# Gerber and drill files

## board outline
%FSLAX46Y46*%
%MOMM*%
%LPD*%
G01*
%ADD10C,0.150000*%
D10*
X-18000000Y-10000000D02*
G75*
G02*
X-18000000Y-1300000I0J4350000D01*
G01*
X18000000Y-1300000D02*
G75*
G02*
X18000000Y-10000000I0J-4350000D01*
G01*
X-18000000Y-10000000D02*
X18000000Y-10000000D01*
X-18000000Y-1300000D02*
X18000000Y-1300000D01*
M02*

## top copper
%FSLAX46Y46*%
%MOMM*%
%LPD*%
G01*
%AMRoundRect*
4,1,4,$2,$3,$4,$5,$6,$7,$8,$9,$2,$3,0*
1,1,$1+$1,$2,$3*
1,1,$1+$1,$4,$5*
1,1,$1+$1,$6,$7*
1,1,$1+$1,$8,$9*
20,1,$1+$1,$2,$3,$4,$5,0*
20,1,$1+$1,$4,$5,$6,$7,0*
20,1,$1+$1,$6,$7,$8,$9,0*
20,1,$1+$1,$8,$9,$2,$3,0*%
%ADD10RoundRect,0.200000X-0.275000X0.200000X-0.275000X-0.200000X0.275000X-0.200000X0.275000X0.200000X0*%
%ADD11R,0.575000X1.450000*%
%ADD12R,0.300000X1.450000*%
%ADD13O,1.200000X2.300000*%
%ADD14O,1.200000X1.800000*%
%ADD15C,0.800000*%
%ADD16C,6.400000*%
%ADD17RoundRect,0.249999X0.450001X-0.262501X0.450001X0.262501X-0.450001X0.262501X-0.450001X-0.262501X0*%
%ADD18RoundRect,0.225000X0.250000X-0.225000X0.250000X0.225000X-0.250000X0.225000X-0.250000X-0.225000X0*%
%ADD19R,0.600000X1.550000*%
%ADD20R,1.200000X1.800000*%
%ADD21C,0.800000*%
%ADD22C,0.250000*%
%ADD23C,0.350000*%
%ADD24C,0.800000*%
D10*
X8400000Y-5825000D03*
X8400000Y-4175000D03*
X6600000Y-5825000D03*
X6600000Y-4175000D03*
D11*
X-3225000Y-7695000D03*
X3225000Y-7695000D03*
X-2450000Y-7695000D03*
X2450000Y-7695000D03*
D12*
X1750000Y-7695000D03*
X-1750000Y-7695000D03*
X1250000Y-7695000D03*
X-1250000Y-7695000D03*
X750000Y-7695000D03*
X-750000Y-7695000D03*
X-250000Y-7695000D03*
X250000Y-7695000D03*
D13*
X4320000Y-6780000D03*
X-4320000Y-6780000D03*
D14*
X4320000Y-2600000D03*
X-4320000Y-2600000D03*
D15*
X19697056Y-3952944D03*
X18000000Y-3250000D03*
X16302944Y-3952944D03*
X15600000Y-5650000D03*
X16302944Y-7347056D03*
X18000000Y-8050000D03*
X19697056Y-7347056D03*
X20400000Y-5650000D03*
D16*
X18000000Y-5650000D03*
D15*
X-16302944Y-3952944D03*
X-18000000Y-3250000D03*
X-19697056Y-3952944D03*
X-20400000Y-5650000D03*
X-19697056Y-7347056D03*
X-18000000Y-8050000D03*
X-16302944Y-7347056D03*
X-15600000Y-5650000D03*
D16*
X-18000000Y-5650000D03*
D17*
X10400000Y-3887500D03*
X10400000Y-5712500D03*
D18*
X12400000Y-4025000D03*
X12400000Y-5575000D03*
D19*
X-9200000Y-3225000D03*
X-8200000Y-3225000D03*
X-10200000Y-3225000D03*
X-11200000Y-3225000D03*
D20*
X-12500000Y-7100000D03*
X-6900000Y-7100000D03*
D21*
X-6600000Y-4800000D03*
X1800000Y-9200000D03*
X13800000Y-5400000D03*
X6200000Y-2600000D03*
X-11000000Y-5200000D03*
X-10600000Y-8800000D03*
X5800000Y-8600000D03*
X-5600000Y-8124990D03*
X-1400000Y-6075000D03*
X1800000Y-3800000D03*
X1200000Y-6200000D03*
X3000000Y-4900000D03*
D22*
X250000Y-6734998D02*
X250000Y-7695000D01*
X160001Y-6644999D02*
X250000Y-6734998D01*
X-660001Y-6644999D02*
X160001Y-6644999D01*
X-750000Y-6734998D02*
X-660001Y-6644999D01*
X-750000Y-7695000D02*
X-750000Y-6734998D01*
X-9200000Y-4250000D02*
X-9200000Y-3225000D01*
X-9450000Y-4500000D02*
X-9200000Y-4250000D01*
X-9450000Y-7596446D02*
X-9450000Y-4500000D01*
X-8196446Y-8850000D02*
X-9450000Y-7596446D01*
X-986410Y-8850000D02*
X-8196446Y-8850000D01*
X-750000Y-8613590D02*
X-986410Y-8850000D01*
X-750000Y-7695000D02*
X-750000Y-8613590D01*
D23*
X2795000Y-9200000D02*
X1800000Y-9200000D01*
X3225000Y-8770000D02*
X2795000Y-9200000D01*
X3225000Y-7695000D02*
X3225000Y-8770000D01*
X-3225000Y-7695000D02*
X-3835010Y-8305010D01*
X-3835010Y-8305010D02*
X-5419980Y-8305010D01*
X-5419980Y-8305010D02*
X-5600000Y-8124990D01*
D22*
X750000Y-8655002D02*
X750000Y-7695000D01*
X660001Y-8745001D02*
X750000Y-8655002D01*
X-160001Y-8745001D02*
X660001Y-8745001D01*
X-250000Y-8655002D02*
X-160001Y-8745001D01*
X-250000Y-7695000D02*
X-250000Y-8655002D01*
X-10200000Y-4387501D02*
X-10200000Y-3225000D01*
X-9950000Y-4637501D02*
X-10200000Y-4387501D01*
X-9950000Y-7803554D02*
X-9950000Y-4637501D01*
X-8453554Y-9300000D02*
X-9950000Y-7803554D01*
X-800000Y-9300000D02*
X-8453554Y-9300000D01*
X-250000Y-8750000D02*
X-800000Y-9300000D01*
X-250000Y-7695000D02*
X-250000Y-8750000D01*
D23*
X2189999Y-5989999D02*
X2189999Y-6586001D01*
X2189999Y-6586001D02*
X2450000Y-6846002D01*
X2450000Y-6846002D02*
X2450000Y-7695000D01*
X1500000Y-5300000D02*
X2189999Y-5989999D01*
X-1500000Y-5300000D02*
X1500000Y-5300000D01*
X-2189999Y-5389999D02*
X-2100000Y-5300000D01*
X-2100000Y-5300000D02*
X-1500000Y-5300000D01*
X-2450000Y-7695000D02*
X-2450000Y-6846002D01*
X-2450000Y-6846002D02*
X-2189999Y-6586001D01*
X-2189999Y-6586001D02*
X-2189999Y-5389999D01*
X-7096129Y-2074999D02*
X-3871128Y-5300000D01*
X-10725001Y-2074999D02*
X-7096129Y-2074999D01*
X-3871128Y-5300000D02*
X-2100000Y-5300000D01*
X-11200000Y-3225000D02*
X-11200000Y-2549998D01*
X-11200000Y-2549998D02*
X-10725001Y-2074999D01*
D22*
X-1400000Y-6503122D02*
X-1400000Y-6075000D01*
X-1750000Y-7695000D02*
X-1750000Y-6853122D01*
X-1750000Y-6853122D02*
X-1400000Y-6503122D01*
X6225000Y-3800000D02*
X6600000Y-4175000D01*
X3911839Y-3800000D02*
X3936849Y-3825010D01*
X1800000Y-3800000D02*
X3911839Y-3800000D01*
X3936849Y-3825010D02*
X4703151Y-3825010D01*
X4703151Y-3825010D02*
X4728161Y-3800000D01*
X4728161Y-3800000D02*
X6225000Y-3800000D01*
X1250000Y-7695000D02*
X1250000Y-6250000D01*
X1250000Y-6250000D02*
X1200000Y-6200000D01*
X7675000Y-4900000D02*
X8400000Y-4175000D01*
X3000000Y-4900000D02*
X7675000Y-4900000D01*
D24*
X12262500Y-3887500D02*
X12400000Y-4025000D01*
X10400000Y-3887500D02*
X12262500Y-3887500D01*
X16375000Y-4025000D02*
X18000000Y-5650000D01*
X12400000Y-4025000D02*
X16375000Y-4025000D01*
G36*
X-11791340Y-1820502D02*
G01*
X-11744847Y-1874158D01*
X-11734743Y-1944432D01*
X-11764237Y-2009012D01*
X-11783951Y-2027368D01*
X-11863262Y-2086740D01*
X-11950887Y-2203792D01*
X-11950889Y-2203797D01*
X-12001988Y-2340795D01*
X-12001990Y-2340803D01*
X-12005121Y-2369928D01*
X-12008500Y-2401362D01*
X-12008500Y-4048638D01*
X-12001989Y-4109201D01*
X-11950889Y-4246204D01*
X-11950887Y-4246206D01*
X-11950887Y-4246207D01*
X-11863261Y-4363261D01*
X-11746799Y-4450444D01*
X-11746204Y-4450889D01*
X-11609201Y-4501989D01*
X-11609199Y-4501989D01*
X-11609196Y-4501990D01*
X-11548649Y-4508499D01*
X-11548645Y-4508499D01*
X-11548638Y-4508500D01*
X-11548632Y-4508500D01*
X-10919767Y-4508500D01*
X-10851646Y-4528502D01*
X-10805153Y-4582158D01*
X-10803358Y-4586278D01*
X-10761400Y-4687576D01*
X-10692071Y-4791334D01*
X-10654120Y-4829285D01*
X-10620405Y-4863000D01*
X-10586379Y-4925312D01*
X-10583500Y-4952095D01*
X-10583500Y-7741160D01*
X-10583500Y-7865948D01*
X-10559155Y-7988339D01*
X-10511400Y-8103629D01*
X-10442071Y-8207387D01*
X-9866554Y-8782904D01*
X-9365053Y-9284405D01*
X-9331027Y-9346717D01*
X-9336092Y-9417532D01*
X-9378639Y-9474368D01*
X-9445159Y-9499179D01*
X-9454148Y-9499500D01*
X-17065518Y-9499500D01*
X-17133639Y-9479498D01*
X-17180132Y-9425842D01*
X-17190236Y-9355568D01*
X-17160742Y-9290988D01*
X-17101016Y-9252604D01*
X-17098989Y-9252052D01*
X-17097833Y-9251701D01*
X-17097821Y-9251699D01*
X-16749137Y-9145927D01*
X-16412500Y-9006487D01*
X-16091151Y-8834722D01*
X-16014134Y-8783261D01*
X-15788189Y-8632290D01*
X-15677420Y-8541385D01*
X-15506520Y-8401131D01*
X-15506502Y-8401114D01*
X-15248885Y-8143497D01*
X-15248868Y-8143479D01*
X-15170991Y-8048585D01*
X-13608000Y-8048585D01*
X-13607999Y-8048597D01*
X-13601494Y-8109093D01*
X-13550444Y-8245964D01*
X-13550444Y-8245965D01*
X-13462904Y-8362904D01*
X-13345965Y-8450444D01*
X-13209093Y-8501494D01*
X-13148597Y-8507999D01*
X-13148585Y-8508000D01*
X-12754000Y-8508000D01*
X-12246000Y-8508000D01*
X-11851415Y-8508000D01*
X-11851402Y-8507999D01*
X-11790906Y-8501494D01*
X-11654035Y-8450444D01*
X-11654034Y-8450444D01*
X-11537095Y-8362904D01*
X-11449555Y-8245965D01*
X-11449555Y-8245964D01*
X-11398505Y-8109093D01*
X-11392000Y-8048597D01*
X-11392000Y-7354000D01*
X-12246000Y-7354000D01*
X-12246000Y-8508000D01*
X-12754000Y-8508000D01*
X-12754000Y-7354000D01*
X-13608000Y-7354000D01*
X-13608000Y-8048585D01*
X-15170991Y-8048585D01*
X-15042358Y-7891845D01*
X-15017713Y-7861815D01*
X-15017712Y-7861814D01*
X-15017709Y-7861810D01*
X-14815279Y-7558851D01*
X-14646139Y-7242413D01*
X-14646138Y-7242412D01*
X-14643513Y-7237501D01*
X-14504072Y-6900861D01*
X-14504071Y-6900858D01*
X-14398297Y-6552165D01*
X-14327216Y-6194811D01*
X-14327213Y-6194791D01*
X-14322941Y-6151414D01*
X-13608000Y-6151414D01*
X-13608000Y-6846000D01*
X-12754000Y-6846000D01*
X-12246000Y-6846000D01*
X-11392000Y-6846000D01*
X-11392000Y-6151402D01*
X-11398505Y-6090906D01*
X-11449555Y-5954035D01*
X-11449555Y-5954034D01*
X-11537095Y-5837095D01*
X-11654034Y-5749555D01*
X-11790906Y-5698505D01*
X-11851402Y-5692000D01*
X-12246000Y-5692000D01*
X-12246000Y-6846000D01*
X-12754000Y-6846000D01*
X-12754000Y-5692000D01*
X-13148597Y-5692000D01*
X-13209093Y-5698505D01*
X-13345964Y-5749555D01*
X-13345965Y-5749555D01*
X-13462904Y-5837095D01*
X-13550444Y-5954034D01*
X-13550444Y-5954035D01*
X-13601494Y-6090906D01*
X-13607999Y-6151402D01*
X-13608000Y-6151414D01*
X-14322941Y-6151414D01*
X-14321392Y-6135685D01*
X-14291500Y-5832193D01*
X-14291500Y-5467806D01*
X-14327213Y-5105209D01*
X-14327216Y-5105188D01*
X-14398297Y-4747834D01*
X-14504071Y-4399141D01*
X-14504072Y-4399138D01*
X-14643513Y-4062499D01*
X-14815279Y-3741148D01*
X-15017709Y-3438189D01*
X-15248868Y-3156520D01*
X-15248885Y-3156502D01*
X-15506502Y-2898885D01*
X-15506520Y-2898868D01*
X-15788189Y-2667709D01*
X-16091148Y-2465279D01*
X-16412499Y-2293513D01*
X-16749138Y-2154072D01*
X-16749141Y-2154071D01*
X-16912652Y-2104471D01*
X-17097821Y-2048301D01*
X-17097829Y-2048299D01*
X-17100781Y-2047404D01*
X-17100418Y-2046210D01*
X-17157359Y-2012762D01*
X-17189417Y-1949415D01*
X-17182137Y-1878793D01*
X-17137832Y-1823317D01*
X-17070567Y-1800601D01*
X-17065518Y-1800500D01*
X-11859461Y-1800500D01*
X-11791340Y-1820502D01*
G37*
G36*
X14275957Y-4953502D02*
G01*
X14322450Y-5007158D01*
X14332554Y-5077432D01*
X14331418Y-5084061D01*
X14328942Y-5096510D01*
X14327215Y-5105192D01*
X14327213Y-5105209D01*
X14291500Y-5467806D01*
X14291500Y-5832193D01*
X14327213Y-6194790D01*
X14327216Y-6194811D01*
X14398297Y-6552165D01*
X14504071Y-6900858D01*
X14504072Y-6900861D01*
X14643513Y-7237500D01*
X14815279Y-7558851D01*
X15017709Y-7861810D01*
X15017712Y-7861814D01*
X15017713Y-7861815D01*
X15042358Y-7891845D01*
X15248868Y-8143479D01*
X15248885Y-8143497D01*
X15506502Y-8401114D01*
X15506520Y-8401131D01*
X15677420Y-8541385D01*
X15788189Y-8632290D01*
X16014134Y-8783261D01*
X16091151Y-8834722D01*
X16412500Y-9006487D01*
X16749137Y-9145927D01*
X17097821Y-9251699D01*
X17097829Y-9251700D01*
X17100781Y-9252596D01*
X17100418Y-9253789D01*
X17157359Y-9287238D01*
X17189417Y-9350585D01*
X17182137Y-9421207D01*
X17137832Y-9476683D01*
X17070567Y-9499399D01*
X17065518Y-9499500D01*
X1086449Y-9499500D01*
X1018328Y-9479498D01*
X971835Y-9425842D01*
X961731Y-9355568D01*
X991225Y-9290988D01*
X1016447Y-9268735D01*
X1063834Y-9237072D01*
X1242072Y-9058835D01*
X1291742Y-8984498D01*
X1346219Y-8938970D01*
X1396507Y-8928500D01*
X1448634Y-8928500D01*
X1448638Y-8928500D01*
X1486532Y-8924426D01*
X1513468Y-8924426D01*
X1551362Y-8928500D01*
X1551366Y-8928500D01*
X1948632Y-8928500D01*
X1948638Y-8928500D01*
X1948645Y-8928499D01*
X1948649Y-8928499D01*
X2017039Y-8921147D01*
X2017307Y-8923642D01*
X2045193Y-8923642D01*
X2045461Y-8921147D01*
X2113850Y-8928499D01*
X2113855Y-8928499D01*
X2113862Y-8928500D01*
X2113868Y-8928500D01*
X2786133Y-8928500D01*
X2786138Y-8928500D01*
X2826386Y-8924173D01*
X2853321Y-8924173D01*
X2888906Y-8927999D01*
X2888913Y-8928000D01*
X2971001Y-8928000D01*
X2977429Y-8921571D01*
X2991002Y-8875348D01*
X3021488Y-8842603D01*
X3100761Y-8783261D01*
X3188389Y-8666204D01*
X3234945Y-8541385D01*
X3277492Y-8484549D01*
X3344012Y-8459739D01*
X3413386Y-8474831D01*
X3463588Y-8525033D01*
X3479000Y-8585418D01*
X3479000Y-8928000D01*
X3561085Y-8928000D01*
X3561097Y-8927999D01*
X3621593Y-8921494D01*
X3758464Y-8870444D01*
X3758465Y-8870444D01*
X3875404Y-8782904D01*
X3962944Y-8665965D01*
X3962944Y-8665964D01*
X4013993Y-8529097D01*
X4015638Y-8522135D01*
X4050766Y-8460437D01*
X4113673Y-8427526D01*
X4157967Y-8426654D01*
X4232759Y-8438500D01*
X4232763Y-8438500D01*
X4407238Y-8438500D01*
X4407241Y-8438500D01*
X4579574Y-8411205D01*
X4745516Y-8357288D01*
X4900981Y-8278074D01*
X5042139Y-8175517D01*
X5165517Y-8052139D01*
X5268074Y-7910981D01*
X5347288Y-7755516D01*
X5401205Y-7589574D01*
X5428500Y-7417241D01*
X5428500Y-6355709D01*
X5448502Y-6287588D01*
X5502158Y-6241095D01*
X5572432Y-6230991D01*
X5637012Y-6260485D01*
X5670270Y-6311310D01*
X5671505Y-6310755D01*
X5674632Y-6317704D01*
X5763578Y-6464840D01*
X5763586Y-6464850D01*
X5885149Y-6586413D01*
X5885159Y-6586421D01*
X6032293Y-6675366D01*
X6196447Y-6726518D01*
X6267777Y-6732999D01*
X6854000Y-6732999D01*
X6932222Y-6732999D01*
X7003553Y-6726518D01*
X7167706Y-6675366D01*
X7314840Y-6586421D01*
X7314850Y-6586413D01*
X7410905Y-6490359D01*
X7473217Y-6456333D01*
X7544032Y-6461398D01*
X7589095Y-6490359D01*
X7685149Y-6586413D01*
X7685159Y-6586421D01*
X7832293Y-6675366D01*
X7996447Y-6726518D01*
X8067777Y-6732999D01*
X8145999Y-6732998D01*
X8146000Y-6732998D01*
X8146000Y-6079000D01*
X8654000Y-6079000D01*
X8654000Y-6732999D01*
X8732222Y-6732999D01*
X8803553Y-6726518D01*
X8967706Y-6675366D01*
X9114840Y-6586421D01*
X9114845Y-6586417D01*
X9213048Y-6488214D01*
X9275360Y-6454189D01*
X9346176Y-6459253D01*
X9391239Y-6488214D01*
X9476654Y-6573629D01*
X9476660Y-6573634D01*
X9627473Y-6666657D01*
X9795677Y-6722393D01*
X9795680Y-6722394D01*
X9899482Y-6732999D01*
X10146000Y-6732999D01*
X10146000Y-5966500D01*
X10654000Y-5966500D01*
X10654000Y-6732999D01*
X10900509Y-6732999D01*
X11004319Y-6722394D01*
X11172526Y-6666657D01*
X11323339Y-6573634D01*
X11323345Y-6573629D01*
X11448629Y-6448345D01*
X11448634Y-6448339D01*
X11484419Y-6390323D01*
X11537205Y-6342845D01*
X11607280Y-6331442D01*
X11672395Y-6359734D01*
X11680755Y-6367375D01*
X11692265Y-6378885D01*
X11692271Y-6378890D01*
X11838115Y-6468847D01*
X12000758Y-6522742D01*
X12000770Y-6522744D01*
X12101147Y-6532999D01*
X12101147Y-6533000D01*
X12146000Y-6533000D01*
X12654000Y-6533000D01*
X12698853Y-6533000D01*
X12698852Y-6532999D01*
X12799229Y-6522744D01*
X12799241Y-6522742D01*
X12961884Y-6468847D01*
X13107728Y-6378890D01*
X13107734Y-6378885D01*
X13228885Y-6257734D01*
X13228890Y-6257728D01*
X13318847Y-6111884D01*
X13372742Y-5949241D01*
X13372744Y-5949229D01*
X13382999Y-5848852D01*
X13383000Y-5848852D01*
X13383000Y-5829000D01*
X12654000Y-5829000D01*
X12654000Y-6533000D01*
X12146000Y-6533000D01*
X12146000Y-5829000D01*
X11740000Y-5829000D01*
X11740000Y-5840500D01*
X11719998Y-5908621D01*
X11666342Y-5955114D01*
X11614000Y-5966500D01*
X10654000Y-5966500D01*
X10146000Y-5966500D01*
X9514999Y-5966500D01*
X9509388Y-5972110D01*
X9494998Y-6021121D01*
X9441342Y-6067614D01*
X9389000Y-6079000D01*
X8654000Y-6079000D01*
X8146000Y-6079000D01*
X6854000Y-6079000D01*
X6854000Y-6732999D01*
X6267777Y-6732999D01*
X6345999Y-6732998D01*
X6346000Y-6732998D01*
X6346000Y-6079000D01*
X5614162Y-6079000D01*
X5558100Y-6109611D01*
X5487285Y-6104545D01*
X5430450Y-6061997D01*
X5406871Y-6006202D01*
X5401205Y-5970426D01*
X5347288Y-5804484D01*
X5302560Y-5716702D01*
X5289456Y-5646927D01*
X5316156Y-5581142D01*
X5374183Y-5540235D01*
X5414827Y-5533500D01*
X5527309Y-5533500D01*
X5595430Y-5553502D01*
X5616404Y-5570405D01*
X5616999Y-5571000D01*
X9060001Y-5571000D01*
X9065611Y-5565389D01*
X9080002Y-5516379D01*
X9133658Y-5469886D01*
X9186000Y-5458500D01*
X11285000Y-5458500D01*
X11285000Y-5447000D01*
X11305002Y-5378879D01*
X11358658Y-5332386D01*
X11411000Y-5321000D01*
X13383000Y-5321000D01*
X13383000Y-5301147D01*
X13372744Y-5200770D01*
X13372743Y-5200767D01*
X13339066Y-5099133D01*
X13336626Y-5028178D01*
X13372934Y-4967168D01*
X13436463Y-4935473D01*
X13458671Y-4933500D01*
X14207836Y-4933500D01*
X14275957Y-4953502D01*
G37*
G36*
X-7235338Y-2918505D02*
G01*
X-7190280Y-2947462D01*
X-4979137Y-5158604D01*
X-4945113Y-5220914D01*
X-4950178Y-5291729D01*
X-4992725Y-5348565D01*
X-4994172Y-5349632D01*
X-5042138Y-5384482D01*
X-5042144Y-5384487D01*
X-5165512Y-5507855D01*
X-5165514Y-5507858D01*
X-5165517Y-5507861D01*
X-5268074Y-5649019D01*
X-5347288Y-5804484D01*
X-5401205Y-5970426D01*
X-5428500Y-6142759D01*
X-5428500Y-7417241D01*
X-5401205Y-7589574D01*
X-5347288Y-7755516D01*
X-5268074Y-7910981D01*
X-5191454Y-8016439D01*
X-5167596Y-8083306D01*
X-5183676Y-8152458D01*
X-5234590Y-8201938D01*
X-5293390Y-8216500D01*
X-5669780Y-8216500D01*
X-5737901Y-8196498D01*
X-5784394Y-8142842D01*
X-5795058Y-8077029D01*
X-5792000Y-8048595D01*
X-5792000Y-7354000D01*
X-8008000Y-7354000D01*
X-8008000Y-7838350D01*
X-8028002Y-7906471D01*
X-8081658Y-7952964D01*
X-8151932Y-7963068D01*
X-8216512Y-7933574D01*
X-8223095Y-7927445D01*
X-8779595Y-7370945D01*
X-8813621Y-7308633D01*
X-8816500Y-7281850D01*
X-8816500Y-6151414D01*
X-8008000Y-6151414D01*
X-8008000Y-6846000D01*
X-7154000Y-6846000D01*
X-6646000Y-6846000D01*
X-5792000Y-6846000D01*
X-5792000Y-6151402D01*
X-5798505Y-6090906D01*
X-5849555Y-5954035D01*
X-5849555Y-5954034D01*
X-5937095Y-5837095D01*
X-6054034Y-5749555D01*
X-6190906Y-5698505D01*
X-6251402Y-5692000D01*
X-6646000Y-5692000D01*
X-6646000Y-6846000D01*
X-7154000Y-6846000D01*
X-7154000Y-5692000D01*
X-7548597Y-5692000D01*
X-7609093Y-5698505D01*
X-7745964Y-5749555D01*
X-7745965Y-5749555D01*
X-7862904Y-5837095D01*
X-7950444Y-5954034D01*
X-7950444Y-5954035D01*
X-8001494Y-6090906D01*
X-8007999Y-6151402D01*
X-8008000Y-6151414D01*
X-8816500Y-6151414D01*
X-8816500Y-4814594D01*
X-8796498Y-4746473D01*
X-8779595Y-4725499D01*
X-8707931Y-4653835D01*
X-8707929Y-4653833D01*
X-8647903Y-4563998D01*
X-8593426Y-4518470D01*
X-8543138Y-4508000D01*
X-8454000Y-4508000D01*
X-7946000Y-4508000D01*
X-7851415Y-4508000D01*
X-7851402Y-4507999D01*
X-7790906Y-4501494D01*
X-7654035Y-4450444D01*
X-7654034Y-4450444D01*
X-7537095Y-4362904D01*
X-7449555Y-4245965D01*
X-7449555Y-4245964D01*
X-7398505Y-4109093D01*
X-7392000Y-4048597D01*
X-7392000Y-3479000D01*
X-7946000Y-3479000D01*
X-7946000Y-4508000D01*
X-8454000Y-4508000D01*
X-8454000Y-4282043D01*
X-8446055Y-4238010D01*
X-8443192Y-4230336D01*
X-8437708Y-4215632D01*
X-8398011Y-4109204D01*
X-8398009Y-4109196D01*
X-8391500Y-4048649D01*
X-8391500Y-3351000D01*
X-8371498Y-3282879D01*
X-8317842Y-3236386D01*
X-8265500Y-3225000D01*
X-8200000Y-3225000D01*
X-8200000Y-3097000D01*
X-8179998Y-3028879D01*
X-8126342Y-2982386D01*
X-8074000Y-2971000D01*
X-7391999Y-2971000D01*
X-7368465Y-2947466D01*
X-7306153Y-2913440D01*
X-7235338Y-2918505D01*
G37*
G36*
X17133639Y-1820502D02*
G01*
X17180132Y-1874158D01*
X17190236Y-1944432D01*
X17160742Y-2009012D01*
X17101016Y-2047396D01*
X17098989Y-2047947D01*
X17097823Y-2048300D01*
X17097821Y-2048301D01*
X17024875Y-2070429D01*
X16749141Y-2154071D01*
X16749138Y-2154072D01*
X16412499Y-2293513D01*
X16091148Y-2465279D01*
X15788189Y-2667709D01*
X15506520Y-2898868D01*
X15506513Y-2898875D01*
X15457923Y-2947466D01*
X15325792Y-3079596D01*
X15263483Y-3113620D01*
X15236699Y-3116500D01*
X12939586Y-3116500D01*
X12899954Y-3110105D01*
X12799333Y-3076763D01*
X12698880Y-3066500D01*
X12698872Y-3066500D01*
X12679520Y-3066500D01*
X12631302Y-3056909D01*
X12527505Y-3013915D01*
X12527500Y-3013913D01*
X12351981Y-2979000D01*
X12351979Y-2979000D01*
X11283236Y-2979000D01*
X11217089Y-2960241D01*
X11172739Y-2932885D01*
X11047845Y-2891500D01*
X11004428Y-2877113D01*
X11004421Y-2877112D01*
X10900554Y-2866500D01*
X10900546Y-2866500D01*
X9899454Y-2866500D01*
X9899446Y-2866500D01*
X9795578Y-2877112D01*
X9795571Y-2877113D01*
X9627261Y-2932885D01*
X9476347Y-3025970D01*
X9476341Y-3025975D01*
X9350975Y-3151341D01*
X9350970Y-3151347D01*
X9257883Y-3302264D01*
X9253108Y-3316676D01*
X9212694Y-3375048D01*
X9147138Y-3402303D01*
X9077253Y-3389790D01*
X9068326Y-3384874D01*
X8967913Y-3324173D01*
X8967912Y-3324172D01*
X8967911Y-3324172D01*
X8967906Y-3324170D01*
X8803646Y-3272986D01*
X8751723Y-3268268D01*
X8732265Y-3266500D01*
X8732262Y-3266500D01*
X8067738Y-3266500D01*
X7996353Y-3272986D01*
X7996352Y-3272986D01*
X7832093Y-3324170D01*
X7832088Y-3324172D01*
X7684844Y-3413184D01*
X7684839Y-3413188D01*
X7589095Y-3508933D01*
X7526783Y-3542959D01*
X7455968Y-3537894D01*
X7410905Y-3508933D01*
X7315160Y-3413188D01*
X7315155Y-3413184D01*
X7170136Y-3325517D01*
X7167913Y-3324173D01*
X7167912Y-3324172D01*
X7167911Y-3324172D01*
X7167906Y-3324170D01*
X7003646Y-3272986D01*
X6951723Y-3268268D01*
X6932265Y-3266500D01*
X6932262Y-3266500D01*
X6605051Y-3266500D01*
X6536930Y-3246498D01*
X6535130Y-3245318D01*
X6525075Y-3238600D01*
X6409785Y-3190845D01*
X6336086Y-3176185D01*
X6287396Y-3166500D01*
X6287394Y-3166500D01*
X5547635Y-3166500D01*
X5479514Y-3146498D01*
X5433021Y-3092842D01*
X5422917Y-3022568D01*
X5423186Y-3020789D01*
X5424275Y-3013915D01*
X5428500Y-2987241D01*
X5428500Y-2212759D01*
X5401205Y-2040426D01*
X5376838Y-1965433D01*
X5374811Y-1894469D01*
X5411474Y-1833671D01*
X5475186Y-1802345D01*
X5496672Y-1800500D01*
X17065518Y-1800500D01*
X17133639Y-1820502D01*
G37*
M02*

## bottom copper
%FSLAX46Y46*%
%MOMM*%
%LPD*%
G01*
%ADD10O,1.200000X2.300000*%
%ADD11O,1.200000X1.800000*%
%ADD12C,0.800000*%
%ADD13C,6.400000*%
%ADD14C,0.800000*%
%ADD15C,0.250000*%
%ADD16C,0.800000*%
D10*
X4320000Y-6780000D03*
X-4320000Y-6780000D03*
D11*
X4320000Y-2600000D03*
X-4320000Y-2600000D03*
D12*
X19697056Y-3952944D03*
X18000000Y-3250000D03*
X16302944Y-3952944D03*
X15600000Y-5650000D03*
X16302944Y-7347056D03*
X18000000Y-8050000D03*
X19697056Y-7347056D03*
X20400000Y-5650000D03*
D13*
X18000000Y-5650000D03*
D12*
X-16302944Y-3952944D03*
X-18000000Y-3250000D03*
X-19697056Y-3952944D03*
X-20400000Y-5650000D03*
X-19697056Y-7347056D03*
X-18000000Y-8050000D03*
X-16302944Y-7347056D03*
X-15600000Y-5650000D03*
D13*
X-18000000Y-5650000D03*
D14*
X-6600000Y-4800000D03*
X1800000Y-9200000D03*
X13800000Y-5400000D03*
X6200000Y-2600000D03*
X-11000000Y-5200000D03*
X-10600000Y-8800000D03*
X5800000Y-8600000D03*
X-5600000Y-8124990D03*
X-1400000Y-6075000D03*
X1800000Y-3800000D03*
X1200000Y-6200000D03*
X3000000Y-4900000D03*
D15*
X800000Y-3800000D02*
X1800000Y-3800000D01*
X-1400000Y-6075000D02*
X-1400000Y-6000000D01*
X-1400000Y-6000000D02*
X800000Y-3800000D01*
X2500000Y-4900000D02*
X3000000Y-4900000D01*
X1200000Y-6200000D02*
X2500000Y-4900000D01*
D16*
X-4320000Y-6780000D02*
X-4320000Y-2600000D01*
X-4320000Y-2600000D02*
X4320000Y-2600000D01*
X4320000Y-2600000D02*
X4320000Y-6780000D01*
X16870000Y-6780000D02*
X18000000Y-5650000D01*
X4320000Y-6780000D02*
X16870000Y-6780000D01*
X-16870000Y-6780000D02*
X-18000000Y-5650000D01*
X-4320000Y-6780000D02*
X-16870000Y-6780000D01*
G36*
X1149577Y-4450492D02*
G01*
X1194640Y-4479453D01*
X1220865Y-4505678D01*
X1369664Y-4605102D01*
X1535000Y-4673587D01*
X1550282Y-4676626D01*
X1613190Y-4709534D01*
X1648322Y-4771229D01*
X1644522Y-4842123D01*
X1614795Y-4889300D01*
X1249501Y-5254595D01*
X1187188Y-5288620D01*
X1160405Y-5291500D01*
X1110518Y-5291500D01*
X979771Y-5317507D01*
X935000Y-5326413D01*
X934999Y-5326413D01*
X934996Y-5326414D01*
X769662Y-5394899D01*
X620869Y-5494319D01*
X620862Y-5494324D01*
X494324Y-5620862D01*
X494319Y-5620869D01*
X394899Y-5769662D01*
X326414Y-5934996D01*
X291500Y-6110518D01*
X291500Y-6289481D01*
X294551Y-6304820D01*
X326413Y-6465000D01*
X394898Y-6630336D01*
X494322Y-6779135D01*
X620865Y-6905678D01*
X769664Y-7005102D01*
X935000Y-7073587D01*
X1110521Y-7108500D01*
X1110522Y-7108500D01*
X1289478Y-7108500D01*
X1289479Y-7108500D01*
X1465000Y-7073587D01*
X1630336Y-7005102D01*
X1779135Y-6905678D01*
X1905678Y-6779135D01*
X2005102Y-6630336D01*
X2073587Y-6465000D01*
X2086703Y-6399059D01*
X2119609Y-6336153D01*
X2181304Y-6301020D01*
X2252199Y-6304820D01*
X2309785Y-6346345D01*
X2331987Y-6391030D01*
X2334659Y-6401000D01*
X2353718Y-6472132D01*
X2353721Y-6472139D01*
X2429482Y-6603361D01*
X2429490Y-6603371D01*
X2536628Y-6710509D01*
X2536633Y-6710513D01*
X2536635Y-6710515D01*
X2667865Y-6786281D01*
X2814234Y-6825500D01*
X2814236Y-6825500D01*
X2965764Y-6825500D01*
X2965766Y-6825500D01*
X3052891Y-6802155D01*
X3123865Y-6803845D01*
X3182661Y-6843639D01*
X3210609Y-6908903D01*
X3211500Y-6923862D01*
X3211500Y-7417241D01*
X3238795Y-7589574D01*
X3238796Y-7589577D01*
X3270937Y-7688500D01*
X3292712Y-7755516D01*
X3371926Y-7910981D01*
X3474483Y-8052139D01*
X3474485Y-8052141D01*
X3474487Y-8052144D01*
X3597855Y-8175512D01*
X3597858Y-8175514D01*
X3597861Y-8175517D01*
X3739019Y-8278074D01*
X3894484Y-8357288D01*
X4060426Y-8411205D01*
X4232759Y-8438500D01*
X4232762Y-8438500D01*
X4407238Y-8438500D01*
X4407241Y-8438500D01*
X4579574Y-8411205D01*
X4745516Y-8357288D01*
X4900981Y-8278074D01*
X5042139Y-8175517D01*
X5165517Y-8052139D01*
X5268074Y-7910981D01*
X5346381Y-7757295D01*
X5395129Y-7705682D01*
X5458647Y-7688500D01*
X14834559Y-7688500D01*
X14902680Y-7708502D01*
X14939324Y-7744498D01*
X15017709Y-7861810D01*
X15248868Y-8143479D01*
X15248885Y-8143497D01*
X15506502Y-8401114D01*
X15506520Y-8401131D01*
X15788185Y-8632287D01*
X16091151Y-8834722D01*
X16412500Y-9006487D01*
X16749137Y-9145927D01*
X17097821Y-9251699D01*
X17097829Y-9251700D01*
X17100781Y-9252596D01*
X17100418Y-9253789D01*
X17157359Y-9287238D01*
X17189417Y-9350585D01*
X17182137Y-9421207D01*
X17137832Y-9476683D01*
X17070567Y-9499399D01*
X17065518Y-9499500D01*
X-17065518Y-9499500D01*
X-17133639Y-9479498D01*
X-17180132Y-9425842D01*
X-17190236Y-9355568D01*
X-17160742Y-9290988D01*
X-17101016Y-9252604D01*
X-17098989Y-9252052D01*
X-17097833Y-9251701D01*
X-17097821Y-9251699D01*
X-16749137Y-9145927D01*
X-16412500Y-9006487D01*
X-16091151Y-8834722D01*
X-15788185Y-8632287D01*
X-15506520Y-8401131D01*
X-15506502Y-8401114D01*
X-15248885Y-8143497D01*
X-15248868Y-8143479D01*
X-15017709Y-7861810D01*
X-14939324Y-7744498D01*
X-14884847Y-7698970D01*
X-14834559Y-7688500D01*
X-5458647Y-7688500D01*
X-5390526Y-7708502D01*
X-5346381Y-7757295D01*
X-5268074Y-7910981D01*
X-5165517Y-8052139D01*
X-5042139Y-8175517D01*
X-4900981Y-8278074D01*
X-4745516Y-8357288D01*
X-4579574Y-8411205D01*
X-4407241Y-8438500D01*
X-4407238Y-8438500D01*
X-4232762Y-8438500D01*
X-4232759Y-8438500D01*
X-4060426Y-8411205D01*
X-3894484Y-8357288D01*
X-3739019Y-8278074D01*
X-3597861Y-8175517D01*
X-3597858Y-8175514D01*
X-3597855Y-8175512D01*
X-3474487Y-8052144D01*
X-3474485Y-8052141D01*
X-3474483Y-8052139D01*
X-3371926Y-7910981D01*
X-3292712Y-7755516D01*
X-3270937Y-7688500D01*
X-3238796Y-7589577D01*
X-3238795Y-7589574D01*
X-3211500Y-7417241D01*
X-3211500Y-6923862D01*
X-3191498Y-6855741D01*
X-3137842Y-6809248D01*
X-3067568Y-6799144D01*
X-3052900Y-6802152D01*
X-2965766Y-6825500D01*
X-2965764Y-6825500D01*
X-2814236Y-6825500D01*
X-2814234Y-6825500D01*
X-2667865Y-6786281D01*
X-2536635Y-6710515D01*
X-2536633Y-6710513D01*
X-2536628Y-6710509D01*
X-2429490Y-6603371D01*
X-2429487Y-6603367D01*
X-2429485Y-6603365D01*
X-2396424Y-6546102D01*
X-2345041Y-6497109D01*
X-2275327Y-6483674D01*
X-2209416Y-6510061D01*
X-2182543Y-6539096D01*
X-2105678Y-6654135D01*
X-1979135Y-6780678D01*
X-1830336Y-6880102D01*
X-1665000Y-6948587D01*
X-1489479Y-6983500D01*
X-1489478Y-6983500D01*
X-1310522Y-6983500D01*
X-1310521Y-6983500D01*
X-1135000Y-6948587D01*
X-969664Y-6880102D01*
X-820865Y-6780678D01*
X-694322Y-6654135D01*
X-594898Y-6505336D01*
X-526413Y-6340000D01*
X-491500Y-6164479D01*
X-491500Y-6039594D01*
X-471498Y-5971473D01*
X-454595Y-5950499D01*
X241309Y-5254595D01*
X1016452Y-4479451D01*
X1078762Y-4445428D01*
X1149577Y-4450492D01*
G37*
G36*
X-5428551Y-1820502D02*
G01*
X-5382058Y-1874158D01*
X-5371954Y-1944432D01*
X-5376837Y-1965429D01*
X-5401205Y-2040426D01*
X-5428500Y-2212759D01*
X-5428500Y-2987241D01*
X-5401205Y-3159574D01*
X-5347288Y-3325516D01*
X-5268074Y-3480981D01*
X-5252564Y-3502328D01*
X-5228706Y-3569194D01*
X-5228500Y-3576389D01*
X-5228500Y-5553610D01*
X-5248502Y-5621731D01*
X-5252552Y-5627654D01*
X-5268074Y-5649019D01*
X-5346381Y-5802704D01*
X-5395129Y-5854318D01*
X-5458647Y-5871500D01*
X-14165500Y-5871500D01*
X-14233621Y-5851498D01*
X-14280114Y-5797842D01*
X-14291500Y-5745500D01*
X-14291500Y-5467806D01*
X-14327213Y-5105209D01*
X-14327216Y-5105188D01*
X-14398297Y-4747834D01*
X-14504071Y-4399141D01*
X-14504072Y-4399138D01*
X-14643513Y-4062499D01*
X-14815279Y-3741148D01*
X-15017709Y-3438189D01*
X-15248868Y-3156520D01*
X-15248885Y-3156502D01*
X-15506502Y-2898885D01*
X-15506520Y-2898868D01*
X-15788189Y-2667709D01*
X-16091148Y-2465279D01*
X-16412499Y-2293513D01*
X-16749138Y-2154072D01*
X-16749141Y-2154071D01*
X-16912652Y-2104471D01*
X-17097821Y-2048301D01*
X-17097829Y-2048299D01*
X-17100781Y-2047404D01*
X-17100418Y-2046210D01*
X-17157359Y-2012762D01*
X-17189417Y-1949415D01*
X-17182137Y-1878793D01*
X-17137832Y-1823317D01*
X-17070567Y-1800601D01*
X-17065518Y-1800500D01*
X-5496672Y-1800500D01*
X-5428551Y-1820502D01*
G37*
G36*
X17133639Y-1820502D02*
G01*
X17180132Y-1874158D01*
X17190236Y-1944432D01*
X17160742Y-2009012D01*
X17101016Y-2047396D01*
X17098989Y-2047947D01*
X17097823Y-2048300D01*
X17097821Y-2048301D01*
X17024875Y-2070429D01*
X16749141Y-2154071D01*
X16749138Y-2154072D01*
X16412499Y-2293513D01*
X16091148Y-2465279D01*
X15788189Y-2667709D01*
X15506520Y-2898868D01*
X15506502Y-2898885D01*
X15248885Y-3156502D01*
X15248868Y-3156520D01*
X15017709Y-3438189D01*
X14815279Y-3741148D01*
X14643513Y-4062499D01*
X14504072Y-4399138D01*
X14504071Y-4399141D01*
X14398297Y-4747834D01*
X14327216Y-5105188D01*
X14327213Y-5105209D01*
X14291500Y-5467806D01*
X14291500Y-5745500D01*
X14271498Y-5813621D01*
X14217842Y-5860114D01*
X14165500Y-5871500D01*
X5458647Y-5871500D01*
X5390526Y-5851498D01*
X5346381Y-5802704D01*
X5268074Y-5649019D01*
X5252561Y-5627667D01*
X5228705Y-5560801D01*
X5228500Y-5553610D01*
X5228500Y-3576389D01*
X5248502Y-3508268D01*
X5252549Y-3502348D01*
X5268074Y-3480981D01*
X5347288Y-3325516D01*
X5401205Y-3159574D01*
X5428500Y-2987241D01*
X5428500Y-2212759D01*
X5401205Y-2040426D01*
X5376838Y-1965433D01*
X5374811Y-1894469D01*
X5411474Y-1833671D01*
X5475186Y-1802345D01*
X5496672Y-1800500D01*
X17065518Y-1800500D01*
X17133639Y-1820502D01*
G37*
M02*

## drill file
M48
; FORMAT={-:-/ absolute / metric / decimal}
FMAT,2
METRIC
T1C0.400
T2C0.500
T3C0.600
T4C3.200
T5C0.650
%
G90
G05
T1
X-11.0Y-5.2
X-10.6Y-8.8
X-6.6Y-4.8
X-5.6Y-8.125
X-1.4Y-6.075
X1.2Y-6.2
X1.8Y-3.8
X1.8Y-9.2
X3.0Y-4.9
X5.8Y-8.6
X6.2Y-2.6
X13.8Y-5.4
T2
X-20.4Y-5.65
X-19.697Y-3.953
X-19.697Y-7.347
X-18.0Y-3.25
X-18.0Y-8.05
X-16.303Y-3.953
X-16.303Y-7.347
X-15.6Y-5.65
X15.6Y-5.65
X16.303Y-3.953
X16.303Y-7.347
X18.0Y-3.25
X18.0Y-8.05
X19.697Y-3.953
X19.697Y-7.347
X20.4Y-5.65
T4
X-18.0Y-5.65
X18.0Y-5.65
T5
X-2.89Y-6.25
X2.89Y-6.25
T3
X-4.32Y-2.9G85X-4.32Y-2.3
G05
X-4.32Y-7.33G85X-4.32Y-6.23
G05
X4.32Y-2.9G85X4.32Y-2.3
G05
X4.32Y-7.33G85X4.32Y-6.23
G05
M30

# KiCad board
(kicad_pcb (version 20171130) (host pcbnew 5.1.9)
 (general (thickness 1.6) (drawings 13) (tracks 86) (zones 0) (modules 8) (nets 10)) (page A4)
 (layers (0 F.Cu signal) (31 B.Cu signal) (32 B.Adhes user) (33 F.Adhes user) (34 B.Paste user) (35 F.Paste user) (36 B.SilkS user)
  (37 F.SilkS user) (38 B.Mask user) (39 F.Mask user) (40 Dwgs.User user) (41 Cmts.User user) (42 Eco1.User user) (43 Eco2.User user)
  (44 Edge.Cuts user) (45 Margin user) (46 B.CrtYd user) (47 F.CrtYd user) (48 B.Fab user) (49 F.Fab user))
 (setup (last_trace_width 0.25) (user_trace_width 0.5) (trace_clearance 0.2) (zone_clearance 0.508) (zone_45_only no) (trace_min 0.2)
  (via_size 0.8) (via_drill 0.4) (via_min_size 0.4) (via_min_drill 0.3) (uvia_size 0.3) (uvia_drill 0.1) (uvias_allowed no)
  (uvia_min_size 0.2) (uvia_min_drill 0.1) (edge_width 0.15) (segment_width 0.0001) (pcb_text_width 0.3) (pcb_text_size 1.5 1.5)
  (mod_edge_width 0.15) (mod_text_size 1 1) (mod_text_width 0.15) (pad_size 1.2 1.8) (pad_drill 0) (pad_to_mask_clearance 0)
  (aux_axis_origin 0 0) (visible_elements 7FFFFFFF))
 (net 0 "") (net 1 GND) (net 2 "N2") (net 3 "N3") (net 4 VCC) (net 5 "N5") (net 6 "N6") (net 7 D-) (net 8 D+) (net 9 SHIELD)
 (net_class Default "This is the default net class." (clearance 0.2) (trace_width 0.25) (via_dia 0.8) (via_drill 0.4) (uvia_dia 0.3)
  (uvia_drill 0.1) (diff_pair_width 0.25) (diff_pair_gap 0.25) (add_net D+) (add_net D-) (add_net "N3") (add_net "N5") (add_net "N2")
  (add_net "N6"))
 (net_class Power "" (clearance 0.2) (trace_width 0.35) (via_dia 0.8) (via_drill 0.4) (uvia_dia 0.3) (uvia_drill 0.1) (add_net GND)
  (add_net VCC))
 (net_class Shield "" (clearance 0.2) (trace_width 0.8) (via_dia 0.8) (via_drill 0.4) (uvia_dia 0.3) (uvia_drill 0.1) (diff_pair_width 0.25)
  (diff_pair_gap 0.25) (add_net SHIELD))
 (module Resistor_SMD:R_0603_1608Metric (layer F.Cu) (at 8.4 5 270)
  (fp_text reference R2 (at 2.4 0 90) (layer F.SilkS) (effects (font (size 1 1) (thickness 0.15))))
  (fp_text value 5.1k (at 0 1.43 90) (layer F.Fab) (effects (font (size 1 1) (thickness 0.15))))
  (pad 2 smd roundrect (at 0.825 0 270) (size 0.8 0.95) (layers F.Cu F.Paste F.Mask) (roundrect_rratio 0.25) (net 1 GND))
  (pad 1 smd roundrect (at -0.825 0 270) (size 0.8 0.95) (layers F.Cu F.Paste F.Mask) (roundrect_rratio 0.25) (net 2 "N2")))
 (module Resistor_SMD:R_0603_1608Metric (layer F.Cu) (at 6.6 5 270)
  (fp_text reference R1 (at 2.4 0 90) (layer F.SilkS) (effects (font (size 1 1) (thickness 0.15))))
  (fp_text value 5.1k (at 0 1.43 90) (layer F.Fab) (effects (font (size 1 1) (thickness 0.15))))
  (pad 2 smd roundrect (at 0.825 0 270) (size 0.8 0.95) (layers F.Cu F.Paste F.Mask) (roundrect_rratio 0.25) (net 1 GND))
  (pad 1 smd roundrect (at -0.825 0 270) (size 0.8 0.95) (layers F.Cu F.Paste F.Mask) (roundrect_rratio 0.25) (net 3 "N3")))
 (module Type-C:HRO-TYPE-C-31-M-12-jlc (layer F.Cu) (at 0 0 180)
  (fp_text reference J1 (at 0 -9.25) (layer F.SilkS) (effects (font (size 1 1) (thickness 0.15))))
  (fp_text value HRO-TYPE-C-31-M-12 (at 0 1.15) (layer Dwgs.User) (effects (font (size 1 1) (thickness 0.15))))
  (pad 12 smd rect (at 3.225 -7.695 180) (size 0.575 1.45) (layers F.Cu F.Paste F.Mask) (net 1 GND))
  (pad 1 smd rect (at -3.225 -7.695 180) (size 0.575 1.45) (layers F.Cu F.Paste F.Mask) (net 1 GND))
  (pad 11 smd rect (at 2.45 -7.695 180) (size 0.575 1.45) (layers F.Cu F.Paste F.Mask) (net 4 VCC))
  (pad 2 smd rect (at -2.45 -7.695 180) (size 0.575 1.45) (layers F.Cu F.Paste F.Mask) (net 4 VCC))
  (pad 3 smd rect (at -1.75 -7.695 180) (size 0.3 1.45) (layers F.Cu F.Paste F.Mask) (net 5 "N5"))
  (pad 10 smd rect (at 1.75 -7.695 180) (size 0.3 1.45) (layers F.Cu F.Paste F.Mask) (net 3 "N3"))
  (pad 4 smd rect (at -1.25 -7.695 180) (size 0.3 1.45) (layers F.Cu F.Paste F.Mask) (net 2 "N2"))
  (pad 9 smd rect (at 1.25 -7.695 180) (size 0.3 1.45) (layers F.Cu F.Paste F.Mask) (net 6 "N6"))
  (pad 5 smd rect (at -0.75 -7.695 180) (size 0.3 1.45) (layers F.Cu F.Paste F.Mask) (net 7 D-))
  (pad 8 smd rect (at 0.75 -7.695 180) (size 0.3 1.45) (layers F.Cu F.Paste F.Mask) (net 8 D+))
  (pad 7 smd rect (at 0.25 -7.695 180) (size 0.3 1.45) (layers F.Cu F.Paste F.Mask) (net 7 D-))
  (pad 6 smd rect (at -0.25 -7.695 180) (size 0.3 1.45) (layers F.Cu F.Paste F.Mask) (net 8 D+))
  (pad "" np_thru_hole circle (at 2.89 -6.25 180) (size 0.65 0.65) (drill 0.65) (layers *.Cu *.Mask))
  (pad "" np_thru_hole circle (at -2.89 -6.25 180) (size 0.65 0.65) (drill 0.65) (layers *.Cu *.Mask))
  (pad 13 thru_hole oval (at -4.32 -6.78 180) (size 1.2 2.3) (drill oval 0.6 1.7) (layers *.Cu *.Mask) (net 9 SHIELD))
  (pad 13 thru_hole oval (at 4.32 -6.78 180) (size 1.2 2.3) (drill oval 0.6 1.7) (layers *.Cu *.Mask) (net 9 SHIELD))
  (pad 13 thru_hole oval (at -4.32 -2.6 180) (size 1.2 1.8) (drill oval 0.6 1.2) (layers *.Cu *.Mask) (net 9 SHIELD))
  (pad 13 thru_hole oval (at 4.32 -2.6 180) (size 1.2 1.8) (drill oval 0.6 1.2) (layers *.Cu *.Mask) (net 9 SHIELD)))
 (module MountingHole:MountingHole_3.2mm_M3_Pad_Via (layer F.Cu) (at 18 5.65)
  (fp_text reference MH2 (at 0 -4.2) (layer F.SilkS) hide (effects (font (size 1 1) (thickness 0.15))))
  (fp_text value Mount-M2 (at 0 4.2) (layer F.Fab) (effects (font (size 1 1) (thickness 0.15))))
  (pad 1 thru_hole circle (at 1.697056 -1.697056) (size 0.8 0.8) (drill 0.5) (layers *.Cu *.Mask) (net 9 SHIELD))
  (pad 1 thru_hole circle (at 0 -2.4) (size 0.8 0.8) (drill 0.5) (layers *.Cu *.Mask) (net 9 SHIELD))
  (pad 1 thru_hole circle (at -1.697056 -1.697056) (size 0.8 0.8) (drill 0.5) (layers *.Cu *.Mask) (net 9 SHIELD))
  (pad 1 thru_hole circle (at -2.4 0) (size 0.8 0.8) (drill 0.5) (layers *.Cu *.Mask) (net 9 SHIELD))
  (pad 1 thru_hole circle (at -1.697056 1.697056) (size 0.8 0.8) (drill 0.5) (layers *.Cu *.Mask) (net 9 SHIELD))
  (pad 1 thru_hole circle (at 0 2.4) (size 0.8 0.8) (drill 0.5) (layers *.Cu *.Mask) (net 9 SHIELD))
  (pad 1 thru_hole circle (at 1.697056 1.697056) (size 0.8 0.8) (drill 0.5) (layers *.Cu *.Mask) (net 9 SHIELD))
  (pad 1 thru_hole circle (at 2.4 0) (size 0.8 0.8) (drill 0.5) (layers *.Cu *.Mask) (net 9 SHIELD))
  (pad 1 thru_hole circle (at 0 0) (size 6.4 6.4) (drill 3.2) (layers *.Cu *.Mask) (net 9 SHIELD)))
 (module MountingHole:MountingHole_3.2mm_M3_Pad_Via (layer F.Cu) (at -18 5.65)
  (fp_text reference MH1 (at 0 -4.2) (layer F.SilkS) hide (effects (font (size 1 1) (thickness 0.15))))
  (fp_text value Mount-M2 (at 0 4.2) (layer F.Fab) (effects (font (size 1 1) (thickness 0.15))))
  (pad 1 thru_hole circle (at 1.697056 -1.697056) (size 0.8 0.8) (drill 0.5) (layers *.Cu *.Mask) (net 9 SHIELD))
  (pad 1 thru_hole circle (at 0 -2.4) (size 0.8 0.8) (drill 0.5) (layers *.Cu *.Mask) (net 9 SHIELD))
  (pad 1 thru_hole circle (at -1.697056 -1.697056) (size 0.8 0.8) (drill 0.5) (layers *.Cu *.Mask) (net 9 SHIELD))
  (pad 1 thru_hole circle (at -2.4 0) (size 0.8 0.8) (drill 0.5) (layers *.Cu *.Mask) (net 9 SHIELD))
  (pad 1 thru_hole circle (at -1.697056 1.697056) (size 0.8 0.8) (drill 0.5) (layers *.Cu *.Mask) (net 9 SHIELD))
  (pad 1 thru_hole circle (at 0 2.4) (size 0.8 0.8) (drill 0.5) (layers *.Cu *.Mask) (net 9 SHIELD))
  (pad 1 thru_hole circle (at 1.697056 1.697056) (size 0.8 0.8) (drill 0.5) (layers *.Cu *.Mask) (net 9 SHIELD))
  (pad 1 thru_hole circle (at 2.4 0) (size 0.8 0.8) (drill 0.5) (layers *.Cu *.Mask) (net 9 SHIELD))
  (pad 1 thru_hole circle (at 0 0) (size 6.4 6.4) (drill 3.2) (layers *.Cu *.Mask) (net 9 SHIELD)))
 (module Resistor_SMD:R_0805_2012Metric (layer F.Cu) (at 10.4 4.8 90)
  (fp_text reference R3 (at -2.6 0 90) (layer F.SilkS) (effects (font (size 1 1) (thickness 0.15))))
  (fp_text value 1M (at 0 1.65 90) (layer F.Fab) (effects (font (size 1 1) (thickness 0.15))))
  (pad 2 smd roundrect (at 0.9125 0 90) (size 1.025 1.4) (layers F.Cu F.Paste F.Mask) (roundrect_rratio 0.2439014634146341) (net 9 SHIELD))
  (pad 1 smd roundrect (at -0.9125 0 90) (size 1.025 1.4) (layers F.Cu F.Paste F.Mask) (roundrect_rratio 0.2439014634146341) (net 1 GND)))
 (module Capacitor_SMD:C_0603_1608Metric (layer F.Cu) (at 12.4 4.8 90)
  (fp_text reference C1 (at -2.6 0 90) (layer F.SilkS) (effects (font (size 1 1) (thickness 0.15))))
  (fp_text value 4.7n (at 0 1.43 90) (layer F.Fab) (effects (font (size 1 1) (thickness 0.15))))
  (pad 2 smd roundrect (at 0.775 0 90) (size 0.9 0.95) (layers F.Cu F.Paste F.Mask) (roundrect_rratio 0.25) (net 9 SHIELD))
  (pad 1 smd roundrect (at -0.775 0 90) (size 0.9 0.95) (layers F.Cu F.Paste F.Mask) (roundrect_rratio 0.25) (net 1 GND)))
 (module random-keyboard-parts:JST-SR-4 (layer F.Cu) (at -9.7 8)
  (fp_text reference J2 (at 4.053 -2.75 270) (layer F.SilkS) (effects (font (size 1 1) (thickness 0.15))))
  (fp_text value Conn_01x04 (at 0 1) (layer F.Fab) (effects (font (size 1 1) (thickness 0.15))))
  (pad 3 smd rect (at 0.5 -4.775) (size 0.6 1.55) (layers F.Cu F.Paste F.Mask) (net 8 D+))
  (pad 4 smd rect (at 1.5 -4.775) (size 0.6 1.55) (layers F.Cu F.Paste F.Mask) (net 1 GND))
  (pad 2 smd rect (at -0.5 -4.775) (size 0.6 1.55) (layers F.Cu F.Paste F.Mask) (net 7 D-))
  (pad 1 smd rect (at -1.5 -4.775) (size 0.6 1.55) (layers F.Cu F.Paste F.Mask) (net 4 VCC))
  (pad MP smd rect (at -2.8 -0.9) (size 1.2 1.8) (layers F.Cu F.Paste F.Mask) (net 1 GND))
  (pad MP smd rect (at 2.8 -0.9) (size 1.2 1.8) (layers F.Cu F.Paste F.Mask) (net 1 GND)))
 (gr_arc (start -18 5.65) (end -18 1.3) (angle -180) (layer Edge.Cuts) (width 0.15))
 (gr_arc (start 18 5.65) (end 18 10) (angle -180) (layer Edge.Cuts) (width 0.15))
 (gr_line (start -18 10) (end 18 10) (layer Edge.Cuts) (width 0.15))
 (gr_line (start -18 1.3) (end 18 1.3) (layer Edge.Cuts) (width 0.15))
 (segment (start 0.25 6.734998) (end 0.25 7.695) (width 0.25) (layer F.Cu) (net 8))
 (segment (start 0.160001 6.644999) (end 0.25 6.734998) (width 0.25) (layer F.Cu) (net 8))
 (segment (start -0.660001 6.644999) (end 0.160001 6.644999) (width 0.25) (layer F.Cu) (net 8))
 (segment (start -0.75 6.734998) (end -0.660001 6.644999) (width 0.25) (layer F.Cu) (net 8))
 (segment (start -0.75 7.695) (end -0.75 6.734998) (width 0.25) (layer F.Cu) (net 8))
 (segment (start -9.2 4.25) (end -9.2 3.225) (width 0.25) (layer F.Cu) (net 8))
 (segment (start -9.45 4.5) (end -9.2 4.25) (width 0.25) (layer F.Cu) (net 8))
 (segment (start -9.45 7.596446) (end -9.45 4.5) (width 0.25) (layer F.Cu) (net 8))
 (segment (start -8.196446 8.85) (end -9.45 7.596446) (width 0.25) (layer F.Cu) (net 8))
 (segment (start -0.98641 8.85) (end -8.196446 8.85) (width 0.25) (layer F.Cu) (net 8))
 (segment (start -0.75 8.61359) (end -0.98641 8.85) (width 0.25) (layer F.Cu) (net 8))
 (segment (start -0.75 7.695) (end -0.75 8.61359) (width 0.25) (layer F.Cu) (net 8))
 (via (at -6.6 4.8) (size 0.8) (drill 0.4) (layers F.Cu B.Cu) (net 1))
 (via (at 1.8 9.2) (size 0.8) (drill 0.4) (layers F.Cu B.Cu) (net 1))
 (segment (start 2.795 9.2) (end 1.8 9.2) (width 0.35) (layer F.Cu) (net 1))
 (segment (start 3.225 8.77) (end 2.795 9.2) (width 0.35) (layer F.Cu) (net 1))
 (segment (start 3.225 7.695) (end 3.225 8.77) (width 0.35) (layer F.Cu) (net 1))
 (via (at 13.8 5.4) (size 0.8) (drill 0.4) (layers F.Cu B.Cu) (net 1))
 (via (at 6.2 2.6) (size 0.8) (drill 0.4) (layers F.Cu B.Cu) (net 1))
 (via (at -11 5.2) (size 0.8) (drill 0.4) (layers F.Cu B.Cu) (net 1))
 (via (at -10.6 8.8) (size 0.8) (drill 0.4) (layers F.Cu B.Cu) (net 1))
 (via (at 5.8 8.6) (size 0.8) (drill 0.4) (layers F.Cu B.Cu) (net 1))
 (segment (start -3.225 7.695) (end -3.83501 8.30501) (width 0.35) (layer F.Cu) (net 1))
 (segment (start -3.83501 8.30501) (end -5.41998 8.30501) (width 0.35) (layer F.Cu) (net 1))
 (via (at -5.6 8.12499) (size 0.8) (drill 0.4) (layers F.Cu B.Cu) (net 1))
 (segment (start -5.41998 8.30501) (end -5.6 8.12499) (width 0.35) (layer F.Cu) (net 1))
 (segment (start 0.75 8.655002) (end 0.75 7.695) (width 0.25) (layer F.Cu) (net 7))
 (segment (start 0.660001 8.745001) (end 0.75 8.655002) (width 0.25) (layer F.Cu) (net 7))
 (segment (start -0.160001 8.745001) (end 0.660001 8.745001) (width 0.25) (layer F.Cu) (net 7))
 (segment (start -0.25 8.655002) (end -0.160001 8.745001) (width 0.25) (layer F.Cu) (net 7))
 (segment (start -0.25 7.695) (end -0.25 8.655002) (width 0.25) (layer F.Cu) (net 7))
 (segment (start -10.2 4.387501) (end -10.2 3.225) (width 0.25) (layer F.Cu) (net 7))
 (segment (start -9.95 4.637501) (end -10.2 4.387501) (width 0.25) (layer F.Cu) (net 7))
 (segment (start -9.95 7.803554) (end -9.95 4.637501) (width 0.25) (layer F.Cu) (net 7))
 (segment (start -8.453554 9.3) (end -9.95 7.803554) (width 0.25) (layer F.Cu) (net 7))
 (segment (start -0.8 9.3) (end -8.453554 9.3) (width 0.25) (layer F.Cu) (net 7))
 (segment (start -0.25 8.75) (end -0.8 9.3) (width 0.25) (layer F.Cu) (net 7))
 (segment (start -0.25 7.695) (end -0.25 8.75) (width 0.25) (layer F.Cu) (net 7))
 (segment (start 2.189999 5.989999) (end 2.189999 6.586001) (width 0.35) (layer F.Cu) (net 4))
 (segment (start 2.189999 6.586001) (end 2.45 6.846002) (width 0.35) (layer F.Cu) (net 4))
 (segment (start 2.45 6.846002) (end 2.45 7.695) (width 0.35) (layer F.Cu) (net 4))
 (segment (start 1.5 5.3) (end 2.189999 5.989999) (width 0.35) (layer F.Cu) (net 4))
 (segment (start -1.5 5.3) (end 1.5 5.3) (width 0.35) (layer F.Cu) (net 4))
 (segment (start -2.189999 5.389999) (end -2.1 5.3) (width 0.35) (layer F.Cu) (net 4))
 (segment (start -2.1 5.3) (end -1.5 5.3) (width 0.35) (layer F.Cu) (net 4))
 (segment (start -2.45 7.695) (end -2.45 6.846002) (width 0.35) (layer F.Cu) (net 4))
 (segment (start -2.45 6.846002) (end -2.189999 6.586001) (width 0.35) (layer F.Cu) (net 4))
 (segment (start -2.189999 6.586001) (end -2.189999 5.389999) (width 0.35) (layer F.Cu) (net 4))
 (segment (start -7.096129 2.074999) (end -3.871128 5.3) (width 0.35) (layer F.Cu) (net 4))
 (segment (start -10.725001 2.074999) (end -7.096129 2.074999) (width 0.35) (layer F.Cu) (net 4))
 (segment (start -3.871128 5.3) (end -2.1 5.3) (width 0.35) (layer F.Cu) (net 4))
 (segment (start -11.2 3.225) (end -11.2 2.549998) (width 0.35) (layer F.Cu) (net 4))
 (segment (start -11.2 2.549998) (end -10.725001 2.074999) (width 0.35) (layer F.Cu) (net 4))
 (via (at -1.4 6.075) (size 0.8) (drill 0.4) (layers F.Cu B.Cu) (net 3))
 (segment (start -1.4 6.503122) (end -1.4 6.075) (width 0.25) (layer F.Cu) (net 3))
 (segment (start -1.75 7.695) (end -1.75 6.853122) (width 0.25) (layer F.Cu) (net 3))
 (segment (start -1.75 6.853122) (end -1.4 6.503122) (width 0.25) (layer F.Cu) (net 3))
 (via (at 1.8 3.8) (size 0.8) (drill 0.4) (layers F.Cu B.Cu) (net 3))
 (segment (start 0.8 3.8) (end 1.8 3.8) (width 0.25) (layer B.Cu) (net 3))
 (segment (start -1.4 6.075) (end -1.4 6) (width 0.25) (layer B.Cu) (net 3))
 (segment (start -1.4 6) (end 0.8 3.8) (width 0.25) (layer B.Cu) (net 3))
 (segment (start 6.225 3.8) (end 6.6 4.175) (width 0.25) (layer F.Cu) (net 3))
 (segment (start 3.911839 3.8) (end 3.936849 3.82501) (width 0.25) (layer F.Cu) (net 3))
 (segment (start 1.8 3.8) (end 3.911839 3.8) (width 0.25) (layer F.Cu) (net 3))
 (segment (start 3.936849 3.82501) (end 4.703151 3.82501) (width 0.25) (layer F.Cu) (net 3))
 (segment (start 4.703151 3.82501) (end 4.728161 3.8) (width 0.25) (layer F.Cu) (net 3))
 (segment (start 4.728161 3.8) (end 6.225 3.8) (width 0.25) (layer F.Cu) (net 3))
 (segment (start 1.25 7.695) (end 1.25 6.25) (width 0.25) (layer F.Cu) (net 2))
 (via (at 1.2 6.2) (size 0.8) (drill 0.4) (layers F.Cu B.Cu) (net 2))
 (segment (start 1.25 6.25) (end 1.2 6.2) (width 0.25) (layer F.Cu) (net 2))
 (via (at 3 4.9) (size 0.8) (drill 0.4) (layers F.Cu B.Cu) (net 2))
 (segment (start 7.675 4.9) (end 8.4 4.175) (width 0.25) (layer F.Cu) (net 2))
 (segment (start 3 4.9) (end 7.675 4.9) (width 0.25) (layer F.Cu) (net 2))
 (segment (start 2.5 4.9) (end 3 4.9) (width 0.25) (layer B.Cu) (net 2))
 (segment (start 1.2 6.2) (end 2.5 4.9) (width 0.25) (layer B.Cu) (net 2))
 (segment (start -4.32 6.78) (end -4.32 2.6) (width 0.8) (layer B.Cu) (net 9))
 (segment (start -4.32 2.6) (end 4.32 2.6) (width 0.8) (layer B.Cu) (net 9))
 (segment (start 4.32 2.6) (end 4.32 6.78) (width 0.8) (layer B.Cu) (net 9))
 (segment (start 16.87 6.78) (end 18 5.65) (width 0.8) (layer B.Cu) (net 9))
 (segment (start 4.32 6.78) (end 16.87 6.78) (width 0.8) (layer B.Cu) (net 9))
 (segment (start -16.87 6.78) (end -18 5.65) (width 0.8) (layer B.Cu) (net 9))
 (segment (start -4.32 6.78) (end -16.87 6.78) (width 0.8) (layer B.Cu) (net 9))
 (segment (start 12.2625 3.8875) (end 12.4 4.025) (width 0.8) (layer F.Cu) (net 9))
 (segment (start 10.4 3.8875) (end 12.2625 3.8875) (width 0.8) (layer F.Cu) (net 9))
 (segment (start 16.375 4.025) (end 18 5.65) (width 0.8) (layer F.Cu) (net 9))
 (segment (start 12.4 4.025) (end 16.375 4.025) (width 0.8) (layer F.Cu) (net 9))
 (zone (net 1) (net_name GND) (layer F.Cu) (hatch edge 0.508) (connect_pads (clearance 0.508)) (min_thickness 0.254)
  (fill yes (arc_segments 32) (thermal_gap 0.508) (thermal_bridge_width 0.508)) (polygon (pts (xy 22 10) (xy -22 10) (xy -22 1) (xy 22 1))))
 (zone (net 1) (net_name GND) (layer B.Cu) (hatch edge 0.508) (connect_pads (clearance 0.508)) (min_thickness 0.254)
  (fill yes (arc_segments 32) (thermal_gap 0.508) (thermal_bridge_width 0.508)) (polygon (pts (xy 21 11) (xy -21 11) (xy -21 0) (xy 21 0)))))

